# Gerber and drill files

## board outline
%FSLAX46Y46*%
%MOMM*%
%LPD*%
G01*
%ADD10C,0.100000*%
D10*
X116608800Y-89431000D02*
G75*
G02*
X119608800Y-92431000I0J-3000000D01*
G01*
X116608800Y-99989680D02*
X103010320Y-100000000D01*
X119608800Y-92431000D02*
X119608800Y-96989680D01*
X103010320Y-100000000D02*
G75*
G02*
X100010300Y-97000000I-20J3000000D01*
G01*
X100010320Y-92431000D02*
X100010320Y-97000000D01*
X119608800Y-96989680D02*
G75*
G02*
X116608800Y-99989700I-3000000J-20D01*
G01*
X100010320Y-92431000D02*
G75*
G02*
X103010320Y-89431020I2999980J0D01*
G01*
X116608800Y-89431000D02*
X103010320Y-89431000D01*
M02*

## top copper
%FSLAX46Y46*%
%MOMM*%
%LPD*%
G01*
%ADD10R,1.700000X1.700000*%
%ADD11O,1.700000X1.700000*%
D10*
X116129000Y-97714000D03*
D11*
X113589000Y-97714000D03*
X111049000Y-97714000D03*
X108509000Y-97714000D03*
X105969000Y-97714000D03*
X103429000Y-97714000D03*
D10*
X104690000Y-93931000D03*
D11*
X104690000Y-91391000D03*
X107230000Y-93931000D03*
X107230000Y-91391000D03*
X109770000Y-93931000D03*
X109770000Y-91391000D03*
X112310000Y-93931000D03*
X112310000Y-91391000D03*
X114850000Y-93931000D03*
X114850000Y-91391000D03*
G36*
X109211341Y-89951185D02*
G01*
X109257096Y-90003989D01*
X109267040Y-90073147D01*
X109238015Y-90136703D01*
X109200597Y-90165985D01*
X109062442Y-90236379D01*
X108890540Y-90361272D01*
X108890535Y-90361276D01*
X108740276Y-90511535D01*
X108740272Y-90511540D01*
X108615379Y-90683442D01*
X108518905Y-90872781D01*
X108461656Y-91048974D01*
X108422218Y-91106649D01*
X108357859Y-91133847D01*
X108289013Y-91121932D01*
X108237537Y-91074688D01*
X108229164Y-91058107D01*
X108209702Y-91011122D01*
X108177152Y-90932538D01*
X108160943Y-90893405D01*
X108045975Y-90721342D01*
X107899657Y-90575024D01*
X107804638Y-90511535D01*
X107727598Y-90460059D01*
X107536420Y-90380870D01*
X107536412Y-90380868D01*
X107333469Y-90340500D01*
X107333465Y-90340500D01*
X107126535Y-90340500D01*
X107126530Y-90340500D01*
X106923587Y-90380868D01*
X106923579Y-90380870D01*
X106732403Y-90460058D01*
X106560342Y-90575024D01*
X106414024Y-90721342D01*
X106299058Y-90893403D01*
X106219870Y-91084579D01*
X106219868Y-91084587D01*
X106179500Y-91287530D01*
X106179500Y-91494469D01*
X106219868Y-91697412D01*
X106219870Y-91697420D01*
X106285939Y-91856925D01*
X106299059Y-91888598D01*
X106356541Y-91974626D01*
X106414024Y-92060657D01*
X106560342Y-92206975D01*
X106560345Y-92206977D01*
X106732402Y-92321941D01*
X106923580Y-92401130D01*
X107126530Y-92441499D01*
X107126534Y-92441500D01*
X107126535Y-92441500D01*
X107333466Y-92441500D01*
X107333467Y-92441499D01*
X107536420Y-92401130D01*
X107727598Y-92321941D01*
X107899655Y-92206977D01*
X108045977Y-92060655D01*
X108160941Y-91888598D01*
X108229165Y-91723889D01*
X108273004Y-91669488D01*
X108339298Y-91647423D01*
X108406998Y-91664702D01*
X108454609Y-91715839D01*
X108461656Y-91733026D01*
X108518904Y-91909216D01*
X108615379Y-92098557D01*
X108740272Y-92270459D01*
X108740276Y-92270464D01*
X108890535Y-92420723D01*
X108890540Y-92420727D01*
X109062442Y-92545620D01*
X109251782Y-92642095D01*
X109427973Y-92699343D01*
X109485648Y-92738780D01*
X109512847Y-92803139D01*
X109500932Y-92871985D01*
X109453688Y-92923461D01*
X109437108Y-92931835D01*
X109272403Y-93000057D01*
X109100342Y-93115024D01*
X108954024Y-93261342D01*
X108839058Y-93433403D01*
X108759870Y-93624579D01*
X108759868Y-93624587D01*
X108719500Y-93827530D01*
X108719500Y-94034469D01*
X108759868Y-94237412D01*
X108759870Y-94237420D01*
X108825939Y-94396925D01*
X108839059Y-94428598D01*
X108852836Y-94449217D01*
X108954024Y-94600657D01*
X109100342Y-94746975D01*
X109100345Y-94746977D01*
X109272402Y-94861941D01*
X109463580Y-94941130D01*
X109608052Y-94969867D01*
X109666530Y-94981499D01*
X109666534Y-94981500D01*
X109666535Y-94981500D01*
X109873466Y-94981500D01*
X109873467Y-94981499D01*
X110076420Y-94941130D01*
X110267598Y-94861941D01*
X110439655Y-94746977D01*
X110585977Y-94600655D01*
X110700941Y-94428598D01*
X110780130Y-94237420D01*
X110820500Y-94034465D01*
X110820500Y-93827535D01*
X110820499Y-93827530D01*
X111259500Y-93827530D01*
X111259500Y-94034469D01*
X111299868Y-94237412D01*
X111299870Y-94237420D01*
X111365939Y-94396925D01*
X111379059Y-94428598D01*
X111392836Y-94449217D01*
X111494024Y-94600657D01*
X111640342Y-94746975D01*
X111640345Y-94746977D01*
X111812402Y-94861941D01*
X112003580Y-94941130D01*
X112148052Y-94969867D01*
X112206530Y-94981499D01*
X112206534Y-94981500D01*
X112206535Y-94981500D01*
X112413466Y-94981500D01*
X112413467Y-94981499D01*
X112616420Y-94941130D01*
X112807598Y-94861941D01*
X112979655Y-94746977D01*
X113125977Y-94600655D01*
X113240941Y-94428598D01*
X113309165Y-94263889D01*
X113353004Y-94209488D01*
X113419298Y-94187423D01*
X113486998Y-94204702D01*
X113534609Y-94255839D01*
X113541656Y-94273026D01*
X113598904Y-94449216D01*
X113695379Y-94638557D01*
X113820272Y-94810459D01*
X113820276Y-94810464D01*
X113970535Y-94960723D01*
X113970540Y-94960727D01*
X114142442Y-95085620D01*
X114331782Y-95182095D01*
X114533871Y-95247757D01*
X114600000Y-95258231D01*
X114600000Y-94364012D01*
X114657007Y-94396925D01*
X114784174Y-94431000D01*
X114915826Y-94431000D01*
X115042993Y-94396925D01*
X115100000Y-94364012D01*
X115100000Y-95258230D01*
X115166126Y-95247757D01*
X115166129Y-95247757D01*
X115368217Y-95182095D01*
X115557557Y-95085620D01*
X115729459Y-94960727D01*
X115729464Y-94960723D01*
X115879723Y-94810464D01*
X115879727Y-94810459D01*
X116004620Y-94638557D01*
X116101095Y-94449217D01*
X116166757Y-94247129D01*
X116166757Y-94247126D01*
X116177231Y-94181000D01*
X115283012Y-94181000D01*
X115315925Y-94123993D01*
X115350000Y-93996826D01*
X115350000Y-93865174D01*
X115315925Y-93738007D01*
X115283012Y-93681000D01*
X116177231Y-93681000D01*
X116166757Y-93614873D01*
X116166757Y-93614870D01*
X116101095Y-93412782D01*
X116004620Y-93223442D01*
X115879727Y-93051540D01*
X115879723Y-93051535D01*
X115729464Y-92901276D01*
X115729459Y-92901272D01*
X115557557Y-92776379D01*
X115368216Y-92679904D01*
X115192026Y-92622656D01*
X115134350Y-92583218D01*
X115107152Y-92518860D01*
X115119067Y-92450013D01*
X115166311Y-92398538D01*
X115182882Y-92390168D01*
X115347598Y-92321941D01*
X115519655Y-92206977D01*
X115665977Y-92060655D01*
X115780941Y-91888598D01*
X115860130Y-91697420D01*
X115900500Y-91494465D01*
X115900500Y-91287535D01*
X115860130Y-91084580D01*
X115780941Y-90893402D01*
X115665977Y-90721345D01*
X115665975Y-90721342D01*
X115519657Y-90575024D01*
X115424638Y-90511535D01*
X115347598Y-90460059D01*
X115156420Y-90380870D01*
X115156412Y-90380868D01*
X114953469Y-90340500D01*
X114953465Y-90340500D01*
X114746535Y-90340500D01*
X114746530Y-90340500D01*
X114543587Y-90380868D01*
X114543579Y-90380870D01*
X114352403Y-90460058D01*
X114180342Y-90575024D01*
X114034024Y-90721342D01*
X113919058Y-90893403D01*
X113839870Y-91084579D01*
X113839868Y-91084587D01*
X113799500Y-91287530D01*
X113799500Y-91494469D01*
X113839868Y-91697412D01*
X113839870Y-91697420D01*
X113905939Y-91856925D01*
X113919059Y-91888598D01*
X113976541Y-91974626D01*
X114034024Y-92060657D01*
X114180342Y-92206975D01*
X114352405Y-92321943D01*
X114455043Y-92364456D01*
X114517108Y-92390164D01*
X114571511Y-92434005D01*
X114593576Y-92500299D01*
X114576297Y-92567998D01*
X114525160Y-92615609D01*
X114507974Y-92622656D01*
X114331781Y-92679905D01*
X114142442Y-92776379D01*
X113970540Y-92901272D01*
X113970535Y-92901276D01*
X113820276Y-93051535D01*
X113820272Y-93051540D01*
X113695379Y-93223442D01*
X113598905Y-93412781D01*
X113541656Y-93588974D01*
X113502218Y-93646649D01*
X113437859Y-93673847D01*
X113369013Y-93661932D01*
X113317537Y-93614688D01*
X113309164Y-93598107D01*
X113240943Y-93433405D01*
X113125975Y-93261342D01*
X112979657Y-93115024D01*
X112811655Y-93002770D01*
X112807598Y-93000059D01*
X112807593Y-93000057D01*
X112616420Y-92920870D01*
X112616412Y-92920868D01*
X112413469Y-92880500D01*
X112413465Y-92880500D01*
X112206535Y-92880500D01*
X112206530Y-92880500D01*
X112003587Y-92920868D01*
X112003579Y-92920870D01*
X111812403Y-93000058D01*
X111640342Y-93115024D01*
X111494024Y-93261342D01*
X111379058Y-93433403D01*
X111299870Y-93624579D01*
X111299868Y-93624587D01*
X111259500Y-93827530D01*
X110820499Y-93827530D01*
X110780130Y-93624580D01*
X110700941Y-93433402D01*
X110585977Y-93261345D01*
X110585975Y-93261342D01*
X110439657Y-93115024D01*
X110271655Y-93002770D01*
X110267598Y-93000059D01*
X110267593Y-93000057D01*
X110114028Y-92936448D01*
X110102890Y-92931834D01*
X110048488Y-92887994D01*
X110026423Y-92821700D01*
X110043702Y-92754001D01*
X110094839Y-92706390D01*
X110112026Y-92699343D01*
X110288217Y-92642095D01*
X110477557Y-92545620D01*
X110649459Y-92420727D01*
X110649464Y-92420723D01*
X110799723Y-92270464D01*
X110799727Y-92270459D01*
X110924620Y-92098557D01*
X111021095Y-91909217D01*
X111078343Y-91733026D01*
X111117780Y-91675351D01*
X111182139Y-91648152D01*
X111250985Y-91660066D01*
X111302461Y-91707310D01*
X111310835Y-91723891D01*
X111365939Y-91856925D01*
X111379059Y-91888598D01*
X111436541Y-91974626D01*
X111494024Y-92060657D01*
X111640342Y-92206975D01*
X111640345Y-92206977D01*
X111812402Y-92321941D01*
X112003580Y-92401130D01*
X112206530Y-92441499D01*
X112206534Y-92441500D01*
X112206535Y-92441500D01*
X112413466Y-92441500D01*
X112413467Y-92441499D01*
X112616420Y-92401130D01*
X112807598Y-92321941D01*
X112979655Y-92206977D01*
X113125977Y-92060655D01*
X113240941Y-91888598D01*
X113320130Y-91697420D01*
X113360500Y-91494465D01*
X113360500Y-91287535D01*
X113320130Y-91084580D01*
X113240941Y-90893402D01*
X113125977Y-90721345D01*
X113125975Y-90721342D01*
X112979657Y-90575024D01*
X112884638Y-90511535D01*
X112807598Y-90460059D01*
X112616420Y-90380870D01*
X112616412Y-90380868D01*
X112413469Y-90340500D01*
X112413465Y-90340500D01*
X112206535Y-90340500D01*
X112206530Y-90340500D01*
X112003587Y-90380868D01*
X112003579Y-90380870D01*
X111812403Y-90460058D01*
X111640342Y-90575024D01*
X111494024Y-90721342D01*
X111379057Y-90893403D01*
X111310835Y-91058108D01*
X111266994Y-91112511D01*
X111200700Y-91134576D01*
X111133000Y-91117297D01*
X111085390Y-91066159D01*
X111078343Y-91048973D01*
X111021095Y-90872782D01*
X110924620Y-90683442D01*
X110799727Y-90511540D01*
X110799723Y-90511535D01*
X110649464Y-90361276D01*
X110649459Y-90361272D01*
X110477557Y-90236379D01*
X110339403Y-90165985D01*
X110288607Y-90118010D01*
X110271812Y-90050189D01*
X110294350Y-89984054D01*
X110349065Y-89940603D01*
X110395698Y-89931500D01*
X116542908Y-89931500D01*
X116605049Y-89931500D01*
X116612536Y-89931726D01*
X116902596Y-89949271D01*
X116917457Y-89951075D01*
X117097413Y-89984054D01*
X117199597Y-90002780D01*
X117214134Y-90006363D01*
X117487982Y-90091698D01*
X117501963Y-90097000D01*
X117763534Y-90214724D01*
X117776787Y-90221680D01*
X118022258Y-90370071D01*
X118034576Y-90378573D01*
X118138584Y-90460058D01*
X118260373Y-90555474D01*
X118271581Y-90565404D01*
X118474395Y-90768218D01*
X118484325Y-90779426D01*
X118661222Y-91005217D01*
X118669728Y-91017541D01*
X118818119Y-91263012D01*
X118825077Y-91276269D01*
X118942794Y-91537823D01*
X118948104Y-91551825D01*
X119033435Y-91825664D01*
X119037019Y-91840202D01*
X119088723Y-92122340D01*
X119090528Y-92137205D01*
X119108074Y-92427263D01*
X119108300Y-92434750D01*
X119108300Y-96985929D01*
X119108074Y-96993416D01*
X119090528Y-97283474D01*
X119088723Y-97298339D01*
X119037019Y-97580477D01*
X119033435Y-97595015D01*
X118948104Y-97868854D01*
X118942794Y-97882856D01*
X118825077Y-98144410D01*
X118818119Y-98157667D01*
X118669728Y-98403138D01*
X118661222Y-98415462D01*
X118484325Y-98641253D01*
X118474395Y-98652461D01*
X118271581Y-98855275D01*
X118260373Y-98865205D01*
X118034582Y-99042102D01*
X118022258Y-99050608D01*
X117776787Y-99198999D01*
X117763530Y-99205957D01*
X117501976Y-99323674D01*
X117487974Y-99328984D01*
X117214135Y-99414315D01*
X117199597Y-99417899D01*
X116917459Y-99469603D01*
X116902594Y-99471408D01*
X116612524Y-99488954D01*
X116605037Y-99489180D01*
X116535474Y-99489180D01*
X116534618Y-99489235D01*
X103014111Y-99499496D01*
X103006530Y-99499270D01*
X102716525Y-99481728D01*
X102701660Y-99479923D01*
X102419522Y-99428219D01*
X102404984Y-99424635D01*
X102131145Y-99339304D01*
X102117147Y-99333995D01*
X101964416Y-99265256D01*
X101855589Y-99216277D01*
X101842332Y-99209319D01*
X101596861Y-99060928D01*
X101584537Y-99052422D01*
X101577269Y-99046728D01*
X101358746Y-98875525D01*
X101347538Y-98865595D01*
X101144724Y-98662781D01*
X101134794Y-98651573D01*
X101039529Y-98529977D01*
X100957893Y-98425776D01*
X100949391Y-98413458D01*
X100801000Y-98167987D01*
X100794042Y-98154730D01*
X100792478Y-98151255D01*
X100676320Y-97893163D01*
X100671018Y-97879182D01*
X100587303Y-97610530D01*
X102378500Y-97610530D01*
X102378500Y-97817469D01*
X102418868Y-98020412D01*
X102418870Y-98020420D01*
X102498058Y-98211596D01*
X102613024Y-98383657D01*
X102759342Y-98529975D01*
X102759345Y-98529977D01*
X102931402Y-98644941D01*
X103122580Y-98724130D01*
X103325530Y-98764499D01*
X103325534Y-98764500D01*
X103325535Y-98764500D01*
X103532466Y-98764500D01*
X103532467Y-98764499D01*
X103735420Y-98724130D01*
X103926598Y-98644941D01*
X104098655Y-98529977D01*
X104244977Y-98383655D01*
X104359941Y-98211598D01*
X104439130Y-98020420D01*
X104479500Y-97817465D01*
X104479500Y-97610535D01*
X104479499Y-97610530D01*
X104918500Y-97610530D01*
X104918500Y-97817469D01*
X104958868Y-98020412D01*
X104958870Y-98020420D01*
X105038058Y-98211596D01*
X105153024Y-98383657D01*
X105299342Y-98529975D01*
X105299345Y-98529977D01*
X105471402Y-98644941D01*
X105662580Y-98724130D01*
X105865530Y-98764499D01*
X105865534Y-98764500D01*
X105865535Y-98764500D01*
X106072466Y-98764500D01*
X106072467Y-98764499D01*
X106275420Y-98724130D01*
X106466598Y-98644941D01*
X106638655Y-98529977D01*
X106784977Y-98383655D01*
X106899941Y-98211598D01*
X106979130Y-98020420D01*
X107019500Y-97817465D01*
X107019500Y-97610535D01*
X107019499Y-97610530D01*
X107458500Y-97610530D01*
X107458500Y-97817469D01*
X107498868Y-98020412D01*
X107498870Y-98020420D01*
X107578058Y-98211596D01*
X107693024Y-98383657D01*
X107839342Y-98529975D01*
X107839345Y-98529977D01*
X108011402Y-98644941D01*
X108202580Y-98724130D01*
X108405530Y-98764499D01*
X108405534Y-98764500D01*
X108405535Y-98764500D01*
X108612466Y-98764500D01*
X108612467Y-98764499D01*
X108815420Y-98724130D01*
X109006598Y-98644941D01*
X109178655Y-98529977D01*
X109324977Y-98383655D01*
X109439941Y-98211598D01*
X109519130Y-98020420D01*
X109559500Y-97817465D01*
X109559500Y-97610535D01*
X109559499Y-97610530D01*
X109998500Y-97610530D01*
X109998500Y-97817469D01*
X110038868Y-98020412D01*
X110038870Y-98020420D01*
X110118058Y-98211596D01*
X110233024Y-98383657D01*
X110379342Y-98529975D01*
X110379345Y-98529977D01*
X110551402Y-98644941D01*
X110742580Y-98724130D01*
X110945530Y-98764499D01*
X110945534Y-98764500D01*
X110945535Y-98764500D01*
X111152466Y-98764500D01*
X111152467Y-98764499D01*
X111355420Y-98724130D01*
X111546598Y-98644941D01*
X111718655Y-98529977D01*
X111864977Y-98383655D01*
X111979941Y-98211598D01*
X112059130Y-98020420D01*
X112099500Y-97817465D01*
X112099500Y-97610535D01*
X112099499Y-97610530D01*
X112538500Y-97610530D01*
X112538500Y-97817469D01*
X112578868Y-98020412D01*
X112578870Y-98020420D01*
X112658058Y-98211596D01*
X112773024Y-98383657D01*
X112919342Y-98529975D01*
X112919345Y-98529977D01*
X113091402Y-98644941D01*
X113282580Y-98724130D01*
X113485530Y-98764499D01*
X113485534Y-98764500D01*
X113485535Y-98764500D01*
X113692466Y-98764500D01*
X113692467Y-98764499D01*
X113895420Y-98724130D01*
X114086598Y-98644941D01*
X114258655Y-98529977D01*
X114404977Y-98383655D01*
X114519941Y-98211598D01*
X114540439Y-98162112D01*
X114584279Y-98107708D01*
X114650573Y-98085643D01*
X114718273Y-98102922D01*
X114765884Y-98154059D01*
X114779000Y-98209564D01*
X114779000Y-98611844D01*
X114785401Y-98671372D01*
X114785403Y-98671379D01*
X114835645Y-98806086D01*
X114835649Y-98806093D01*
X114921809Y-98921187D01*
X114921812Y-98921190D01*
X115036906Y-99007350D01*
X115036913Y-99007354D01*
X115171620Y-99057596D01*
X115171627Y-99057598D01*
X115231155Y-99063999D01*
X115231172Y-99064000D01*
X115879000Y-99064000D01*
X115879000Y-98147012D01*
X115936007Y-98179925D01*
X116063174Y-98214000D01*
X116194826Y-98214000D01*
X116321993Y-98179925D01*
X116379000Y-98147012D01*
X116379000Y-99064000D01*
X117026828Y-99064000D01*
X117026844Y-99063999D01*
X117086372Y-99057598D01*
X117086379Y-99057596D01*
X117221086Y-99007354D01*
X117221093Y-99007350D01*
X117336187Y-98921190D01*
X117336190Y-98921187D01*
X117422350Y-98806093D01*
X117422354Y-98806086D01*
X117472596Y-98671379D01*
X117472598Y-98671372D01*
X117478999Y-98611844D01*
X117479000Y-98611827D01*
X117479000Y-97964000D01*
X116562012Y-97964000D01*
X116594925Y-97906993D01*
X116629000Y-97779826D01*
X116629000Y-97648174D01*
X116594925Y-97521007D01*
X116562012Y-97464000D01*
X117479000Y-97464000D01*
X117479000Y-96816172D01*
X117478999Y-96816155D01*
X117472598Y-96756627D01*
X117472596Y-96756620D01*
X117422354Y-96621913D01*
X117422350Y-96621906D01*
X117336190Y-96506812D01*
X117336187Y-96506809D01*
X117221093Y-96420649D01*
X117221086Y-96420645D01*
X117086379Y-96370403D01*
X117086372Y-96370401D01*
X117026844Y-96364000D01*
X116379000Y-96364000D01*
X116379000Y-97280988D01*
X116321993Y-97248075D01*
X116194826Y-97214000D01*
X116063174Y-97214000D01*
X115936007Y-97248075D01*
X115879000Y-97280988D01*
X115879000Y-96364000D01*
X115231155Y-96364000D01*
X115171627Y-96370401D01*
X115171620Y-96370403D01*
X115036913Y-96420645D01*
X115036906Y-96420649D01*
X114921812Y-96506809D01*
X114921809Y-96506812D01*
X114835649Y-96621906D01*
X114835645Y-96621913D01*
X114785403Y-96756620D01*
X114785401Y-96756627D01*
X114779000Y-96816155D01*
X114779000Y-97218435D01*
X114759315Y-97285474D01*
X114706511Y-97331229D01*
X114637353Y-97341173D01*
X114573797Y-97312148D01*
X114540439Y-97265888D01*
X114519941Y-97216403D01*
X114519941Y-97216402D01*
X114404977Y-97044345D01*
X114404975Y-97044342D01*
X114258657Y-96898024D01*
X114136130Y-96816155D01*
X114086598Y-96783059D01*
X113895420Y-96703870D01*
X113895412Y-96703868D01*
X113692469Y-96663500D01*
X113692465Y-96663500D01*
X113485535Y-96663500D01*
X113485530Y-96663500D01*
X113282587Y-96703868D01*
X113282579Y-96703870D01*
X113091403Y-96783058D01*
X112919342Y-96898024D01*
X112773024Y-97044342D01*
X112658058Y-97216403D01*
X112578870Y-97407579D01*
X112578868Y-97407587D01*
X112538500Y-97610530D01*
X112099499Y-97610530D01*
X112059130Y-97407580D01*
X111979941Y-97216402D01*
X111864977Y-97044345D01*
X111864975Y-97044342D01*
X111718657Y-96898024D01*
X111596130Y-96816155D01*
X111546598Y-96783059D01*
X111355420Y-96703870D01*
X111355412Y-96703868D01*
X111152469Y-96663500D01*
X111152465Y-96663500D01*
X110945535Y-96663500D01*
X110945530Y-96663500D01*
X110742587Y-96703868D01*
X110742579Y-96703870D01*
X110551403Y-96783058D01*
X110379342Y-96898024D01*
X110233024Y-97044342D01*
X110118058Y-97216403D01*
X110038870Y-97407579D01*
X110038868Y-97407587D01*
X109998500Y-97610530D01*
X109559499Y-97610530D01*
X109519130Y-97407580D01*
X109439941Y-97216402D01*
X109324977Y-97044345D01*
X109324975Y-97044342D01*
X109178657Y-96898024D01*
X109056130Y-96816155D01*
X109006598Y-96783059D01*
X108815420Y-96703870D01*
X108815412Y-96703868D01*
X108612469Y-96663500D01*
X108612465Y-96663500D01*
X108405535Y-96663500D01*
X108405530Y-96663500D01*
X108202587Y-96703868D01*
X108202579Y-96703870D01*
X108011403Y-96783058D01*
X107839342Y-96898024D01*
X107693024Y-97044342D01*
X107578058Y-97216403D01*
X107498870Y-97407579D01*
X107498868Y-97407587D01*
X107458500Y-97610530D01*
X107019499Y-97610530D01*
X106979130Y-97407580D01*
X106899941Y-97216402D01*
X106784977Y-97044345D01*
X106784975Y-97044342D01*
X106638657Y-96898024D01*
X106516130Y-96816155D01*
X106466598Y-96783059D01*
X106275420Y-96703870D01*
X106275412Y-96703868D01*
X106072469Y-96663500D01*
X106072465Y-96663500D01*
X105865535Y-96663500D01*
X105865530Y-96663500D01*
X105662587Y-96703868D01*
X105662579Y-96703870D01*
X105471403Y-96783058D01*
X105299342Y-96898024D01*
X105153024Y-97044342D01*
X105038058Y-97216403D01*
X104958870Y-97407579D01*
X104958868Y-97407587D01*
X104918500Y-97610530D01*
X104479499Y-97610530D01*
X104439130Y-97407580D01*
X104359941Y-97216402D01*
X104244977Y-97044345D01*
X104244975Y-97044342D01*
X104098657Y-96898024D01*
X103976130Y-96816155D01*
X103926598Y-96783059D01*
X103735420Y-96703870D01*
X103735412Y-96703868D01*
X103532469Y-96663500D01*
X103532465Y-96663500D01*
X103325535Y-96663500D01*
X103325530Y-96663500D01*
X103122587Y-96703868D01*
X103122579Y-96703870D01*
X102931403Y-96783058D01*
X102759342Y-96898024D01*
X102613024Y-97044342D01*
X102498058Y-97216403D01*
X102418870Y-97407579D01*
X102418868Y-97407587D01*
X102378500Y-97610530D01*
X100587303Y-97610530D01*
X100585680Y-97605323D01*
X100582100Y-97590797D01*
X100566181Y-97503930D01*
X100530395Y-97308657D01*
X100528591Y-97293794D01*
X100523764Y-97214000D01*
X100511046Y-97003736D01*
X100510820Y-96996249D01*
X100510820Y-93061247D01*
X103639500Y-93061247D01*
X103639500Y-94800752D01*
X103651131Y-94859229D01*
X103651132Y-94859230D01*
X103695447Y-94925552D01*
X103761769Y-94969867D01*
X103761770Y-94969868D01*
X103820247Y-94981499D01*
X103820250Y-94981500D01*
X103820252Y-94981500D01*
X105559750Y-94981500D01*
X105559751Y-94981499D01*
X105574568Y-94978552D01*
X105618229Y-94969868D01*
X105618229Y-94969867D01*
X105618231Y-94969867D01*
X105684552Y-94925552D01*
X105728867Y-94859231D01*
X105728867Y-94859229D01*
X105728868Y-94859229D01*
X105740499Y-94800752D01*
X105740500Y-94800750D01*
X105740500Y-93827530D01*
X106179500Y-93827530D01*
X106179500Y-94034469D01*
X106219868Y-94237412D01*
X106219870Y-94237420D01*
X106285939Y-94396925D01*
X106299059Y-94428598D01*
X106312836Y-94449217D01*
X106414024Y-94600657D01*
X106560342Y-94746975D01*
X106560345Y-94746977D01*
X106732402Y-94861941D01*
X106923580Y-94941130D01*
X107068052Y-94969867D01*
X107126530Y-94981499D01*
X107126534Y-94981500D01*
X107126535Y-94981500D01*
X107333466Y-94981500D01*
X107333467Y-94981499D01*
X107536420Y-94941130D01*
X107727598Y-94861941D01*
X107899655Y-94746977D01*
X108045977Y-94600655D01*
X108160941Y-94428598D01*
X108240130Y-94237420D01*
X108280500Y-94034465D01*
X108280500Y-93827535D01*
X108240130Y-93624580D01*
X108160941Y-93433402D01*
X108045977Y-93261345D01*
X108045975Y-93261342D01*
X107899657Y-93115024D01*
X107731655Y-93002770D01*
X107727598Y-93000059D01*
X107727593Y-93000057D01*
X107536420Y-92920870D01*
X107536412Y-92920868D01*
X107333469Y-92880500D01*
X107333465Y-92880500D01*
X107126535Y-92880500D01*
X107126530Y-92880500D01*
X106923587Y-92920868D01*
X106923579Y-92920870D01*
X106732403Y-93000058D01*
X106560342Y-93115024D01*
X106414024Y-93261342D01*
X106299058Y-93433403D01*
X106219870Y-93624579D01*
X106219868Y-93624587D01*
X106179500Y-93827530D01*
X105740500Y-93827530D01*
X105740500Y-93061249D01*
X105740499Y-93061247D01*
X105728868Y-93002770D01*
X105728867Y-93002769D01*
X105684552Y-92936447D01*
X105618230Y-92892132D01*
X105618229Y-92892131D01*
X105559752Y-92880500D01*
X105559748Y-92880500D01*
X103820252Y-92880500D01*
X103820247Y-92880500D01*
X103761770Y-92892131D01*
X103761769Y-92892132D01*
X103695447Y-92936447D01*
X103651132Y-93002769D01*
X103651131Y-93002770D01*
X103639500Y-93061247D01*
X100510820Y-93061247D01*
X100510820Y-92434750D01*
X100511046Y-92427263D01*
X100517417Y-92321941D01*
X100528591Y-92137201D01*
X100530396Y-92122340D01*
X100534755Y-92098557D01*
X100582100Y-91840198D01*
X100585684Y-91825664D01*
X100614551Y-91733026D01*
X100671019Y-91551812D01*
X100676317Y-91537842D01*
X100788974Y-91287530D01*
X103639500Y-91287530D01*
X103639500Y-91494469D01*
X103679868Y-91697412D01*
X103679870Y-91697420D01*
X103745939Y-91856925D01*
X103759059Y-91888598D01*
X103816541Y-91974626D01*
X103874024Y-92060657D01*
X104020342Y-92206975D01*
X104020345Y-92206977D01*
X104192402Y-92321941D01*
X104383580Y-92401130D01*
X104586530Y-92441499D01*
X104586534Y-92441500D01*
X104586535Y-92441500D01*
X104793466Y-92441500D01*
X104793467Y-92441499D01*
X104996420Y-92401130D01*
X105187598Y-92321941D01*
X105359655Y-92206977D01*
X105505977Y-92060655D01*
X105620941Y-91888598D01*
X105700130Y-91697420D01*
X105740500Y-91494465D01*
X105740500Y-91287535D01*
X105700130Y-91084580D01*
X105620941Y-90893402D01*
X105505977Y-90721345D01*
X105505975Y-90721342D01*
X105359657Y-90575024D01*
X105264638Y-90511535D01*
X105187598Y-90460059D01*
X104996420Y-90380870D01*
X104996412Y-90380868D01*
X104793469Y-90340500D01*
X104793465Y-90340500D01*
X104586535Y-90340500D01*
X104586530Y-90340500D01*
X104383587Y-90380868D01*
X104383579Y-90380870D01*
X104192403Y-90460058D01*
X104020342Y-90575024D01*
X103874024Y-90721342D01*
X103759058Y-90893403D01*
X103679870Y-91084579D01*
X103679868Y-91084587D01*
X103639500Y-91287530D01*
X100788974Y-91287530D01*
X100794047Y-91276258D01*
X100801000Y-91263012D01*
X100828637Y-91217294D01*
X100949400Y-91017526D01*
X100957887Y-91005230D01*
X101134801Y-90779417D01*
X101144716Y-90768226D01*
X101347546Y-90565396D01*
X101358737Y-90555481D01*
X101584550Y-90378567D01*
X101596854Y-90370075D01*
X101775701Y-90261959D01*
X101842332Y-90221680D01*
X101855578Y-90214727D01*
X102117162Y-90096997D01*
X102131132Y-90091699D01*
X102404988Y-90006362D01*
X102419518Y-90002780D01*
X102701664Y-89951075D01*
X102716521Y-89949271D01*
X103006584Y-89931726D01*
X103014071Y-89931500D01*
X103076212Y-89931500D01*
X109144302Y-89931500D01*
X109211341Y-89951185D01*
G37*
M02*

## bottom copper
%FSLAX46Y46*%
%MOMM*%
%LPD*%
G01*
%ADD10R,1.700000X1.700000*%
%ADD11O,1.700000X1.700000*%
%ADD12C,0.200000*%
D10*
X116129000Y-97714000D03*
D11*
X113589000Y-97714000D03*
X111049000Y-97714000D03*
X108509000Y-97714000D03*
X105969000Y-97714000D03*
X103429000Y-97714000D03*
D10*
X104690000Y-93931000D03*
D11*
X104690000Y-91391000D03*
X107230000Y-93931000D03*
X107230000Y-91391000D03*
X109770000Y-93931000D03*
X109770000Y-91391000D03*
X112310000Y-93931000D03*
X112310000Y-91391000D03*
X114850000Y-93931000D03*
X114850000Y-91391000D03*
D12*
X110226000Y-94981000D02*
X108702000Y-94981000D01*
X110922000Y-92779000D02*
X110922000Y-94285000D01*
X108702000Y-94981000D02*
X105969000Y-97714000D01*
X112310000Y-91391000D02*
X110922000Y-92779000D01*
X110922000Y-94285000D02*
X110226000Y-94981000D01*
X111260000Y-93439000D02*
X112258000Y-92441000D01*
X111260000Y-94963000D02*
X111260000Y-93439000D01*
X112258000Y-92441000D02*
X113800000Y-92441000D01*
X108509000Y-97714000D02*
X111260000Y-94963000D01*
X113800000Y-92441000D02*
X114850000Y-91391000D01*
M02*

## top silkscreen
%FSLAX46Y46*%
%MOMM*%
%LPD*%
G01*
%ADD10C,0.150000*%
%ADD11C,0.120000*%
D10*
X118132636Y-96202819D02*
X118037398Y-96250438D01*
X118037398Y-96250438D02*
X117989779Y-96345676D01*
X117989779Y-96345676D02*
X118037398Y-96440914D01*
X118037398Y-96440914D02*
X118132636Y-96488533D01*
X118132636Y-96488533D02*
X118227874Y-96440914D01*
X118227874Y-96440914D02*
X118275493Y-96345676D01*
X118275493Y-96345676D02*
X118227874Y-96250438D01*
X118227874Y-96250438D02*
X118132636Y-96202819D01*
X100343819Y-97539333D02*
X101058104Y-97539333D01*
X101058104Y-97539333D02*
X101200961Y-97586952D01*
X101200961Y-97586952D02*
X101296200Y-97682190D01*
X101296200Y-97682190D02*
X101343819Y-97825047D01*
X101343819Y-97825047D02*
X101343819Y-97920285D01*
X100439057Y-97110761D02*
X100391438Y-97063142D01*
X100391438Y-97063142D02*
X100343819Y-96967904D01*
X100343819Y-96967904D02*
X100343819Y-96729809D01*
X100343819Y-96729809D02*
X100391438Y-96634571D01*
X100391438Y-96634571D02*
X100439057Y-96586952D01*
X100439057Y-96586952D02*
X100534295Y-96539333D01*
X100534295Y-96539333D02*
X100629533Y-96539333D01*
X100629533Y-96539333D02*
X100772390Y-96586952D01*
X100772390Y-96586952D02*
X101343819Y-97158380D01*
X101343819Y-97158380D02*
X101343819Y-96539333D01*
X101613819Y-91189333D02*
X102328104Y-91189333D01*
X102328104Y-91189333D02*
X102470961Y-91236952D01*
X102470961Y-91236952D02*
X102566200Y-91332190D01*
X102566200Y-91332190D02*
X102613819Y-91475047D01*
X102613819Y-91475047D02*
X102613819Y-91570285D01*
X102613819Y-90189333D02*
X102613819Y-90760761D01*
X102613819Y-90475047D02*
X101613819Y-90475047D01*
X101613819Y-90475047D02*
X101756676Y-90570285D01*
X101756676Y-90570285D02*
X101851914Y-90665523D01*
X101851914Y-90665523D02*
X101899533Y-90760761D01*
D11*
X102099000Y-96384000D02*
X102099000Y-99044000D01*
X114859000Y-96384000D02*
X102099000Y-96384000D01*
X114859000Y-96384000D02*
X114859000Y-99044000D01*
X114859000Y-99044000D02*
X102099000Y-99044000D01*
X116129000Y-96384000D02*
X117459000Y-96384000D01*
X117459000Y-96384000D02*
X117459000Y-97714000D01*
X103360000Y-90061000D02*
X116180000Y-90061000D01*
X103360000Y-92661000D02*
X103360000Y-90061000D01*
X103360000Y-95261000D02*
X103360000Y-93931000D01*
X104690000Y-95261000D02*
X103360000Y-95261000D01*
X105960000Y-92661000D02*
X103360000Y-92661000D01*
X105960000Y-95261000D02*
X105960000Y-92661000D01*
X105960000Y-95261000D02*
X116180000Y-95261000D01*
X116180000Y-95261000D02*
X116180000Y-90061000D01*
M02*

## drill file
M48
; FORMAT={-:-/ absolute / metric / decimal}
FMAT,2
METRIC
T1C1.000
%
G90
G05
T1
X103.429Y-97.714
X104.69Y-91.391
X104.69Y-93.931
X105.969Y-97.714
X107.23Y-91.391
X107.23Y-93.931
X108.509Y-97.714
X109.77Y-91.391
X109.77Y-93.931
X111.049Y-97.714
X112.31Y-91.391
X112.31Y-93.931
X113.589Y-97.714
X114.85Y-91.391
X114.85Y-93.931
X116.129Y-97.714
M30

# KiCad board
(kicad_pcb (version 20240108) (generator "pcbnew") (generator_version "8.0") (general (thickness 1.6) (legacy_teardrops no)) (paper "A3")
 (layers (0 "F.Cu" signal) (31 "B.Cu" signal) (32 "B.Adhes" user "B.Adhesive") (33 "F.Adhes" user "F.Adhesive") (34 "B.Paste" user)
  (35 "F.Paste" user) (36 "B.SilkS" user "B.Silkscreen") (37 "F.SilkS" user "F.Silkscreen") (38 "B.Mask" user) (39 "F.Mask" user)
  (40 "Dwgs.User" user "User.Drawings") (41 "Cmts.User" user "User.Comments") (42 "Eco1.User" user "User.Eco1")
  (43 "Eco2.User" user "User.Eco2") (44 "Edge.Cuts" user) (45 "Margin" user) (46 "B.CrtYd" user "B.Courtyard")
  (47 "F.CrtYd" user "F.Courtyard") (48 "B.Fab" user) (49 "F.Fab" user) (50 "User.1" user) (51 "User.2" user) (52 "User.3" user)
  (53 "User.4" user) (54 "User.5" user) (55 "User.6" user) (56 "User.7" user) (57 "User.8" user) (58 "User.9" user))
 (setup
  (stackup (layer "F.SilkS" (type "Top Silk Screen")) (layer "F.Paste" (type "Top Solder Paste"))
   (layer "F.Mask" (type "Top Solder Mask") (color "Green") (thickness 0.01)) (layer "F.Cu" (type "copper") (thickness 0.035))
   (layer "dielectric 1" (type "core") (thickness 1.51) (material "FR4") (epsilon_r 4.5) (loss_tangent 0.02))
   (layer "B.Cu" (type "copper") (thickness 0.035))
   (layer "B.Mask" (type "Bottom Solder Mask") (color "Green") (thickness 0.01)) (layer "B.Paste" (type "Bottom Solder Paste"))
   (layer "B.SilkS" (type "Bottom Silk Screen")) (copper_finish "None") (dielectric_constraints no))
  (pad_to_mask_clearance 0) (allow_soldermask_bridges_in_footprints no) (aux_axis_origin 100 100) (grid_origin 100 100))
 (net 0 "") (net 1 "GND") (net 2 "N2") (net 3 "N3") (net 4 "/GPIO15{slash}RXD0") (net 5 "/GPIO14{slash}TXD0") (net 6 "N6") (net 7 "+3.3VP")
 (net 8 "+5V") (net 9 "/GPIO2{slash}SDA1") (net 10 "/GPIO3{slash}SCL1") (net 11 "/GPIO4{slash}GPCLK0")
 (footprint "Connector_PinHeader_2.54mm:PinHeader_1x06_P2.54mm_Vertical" (layer "F.Cu") (at 116.129 97.714 -90)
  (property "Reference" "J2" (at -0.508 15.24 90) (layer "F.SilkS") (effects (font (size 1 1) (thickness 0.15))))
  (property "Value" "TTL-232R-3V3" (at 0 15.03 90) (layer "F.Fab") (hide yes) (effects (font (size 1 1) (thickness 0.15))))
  (fp_line (start -1.33 14.03) (end 1.33 14.03) (stroke (width 0.12) (type solid)) (layer "F.SilkS"))
  (fp_line (start -1.33 1.27) (end -1.33 14.03) (stroke (width 0.12) (type solid)) (layer "F.SilkS"))
  (fp_line (start -1.33 1.27) (end 1.33 1.27) (stroke (width 0.12) (type solid)) (layer "F.SilkS"))
  (fp_line (start 1.33 1.27) (end 1.33 14.03) (stroke (width 0.12) (type solid)) (layer "F.SilkS"))
  (fp_line (start -1.33 0) (end -1.33 -1.33) (stroke (width 0.12) (type solid)) (layer "F.SilkS"))
  (fp_line (start -1.33 -1.33) (end 0 -1.33) (stroke (width 0.12) (type solid)) (layer "F.SilkS"))
  (pad "1" thru_hole rect (at 0 0 270) (size 1.7 1.7) (drill 1) (layers "*.Cu" "*.Mask") (remove_unused_layers no) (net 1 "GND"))
  (pad "2" thru_hole oval (at 0 2.54 270) (size 1.7 1.7) (drill 1) (layers "*.Cu" "*.Mask") (remove_unused_layers no) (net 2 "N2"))
  (pad "3" thru_hole oval (at 0 5.08 270) (size 1.7 1.7) (drill 1) (layers "*.Cu" "*.Mask") (remove_unused_layers no) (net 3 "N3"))
  (pad "4" thru_hole oval (at 0 7.62 270) (size 1.7 1.7) (drill 1) (layers "*.Cu" "*.Mask") (remove_unused_layers no)
   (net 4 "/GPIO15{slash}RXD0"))
  (pad "5" thru_hole oval (at 0 10.16 270) (size 1.7 1.7) (drill 1) (layers "*.Cu" "*.Mask") (remove_unused_layers no)
   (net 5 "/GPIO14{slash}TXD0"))
  (pad "6" thru_hole oval (at 0 12.7 270) (size 1.7 1.7) (drill 1) (layers "*.Cu" "*.Mask") (remove_unused_layers no) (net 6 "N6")))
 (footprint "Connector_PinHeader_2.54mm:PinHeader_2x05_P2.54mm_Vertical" (layer "F.Cu") (at 104.69 93.931 90)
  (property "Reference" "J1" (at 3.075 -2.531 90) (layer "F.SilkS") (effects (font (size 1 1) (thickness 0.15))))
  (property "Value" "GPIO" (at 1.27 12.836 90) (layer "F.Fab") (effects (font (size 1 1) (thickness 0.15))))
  (fp_line (start 3.87 -1.33) (end 3.87 11.49) (stroke (width 0.12) (type solid)) (layer "F.SilkS"))
  (fp_line (start 1.27 -1.33) (end 3.87 -1.33) (stroke (width 0.12) (type solid)) (layer "F.SilkS"))
  (fp_line (start -1.33 -1.33) (end 0 -1.33) (stroke (width 0.12) (type solid)) (layer "F.SilkS"))
  (fp_line (start -1.33 0) (end -1.33 -1.33) (stroke (width 0.12) (type solid)) (layer "F.SilkS"))
  (fp_line (start 1.27 1.27) (end 1.27 -1.33) (stroke (width 0.12) (type solid)) (layer "F.SilkS"))
  (fp_line (start -1.33 1.27) (end 1.27 1.27) (stroke (width 0.12) (type solid)) (layer "F.SilkS"))
  (fp_line (start -1.33 1.27) (end -1.33 11.49) (stroke (width 0.12) (type solid)) (layer "F.SilkS"))
  (fp_line (start -1.33 11.49) (end 3.87 11.49) (stroke (width 0.12) (type solid)) (layer "F.SilkS"))
  (pad "1" thru_hole rect (at 0 0 90) (size 1.7 1.7) (drill 1) (layers "*.Cu" "*.Mask") (remove_unused_layers no) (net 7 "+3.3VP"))
  (pad "2" thru_hole oval (at 2.54 0 90) (size 1.7 1.7) (drill 1) (layers "*.Cu" "*.Mask") (remove_unused_layers no) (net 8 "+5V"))
  (pad "3" thru_hole oval (at 0 2.54 90) (size 1.7 1.7) (drill 1) (layers "*.Cu" "*.Mask") (remove_unused_layers no)
   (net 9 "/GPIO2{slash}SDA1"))
  (pad "4" thru_hole oval (at 2.54 2.54 90) (size 1.7 1.7) (drill 1) (layers "*.Cu" "*.Mask") (remove_unused_layers no) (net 8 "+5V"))
  (pad "5" thru_hole oval (at 0 5.08 90) (size 1.7 1.7) (drill 1) (layers "*.Cu" "*.Mask") (remove_unused_layers no)
   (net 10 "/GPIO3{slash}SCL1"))
  (pad "6" thru_hole oval (at 2.54 5.08 90) (size 1.7 1.7) (drill 1) (layers "*.Cu" "*.Mask") (remove_unused_layers no) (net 1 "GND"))
  (pad "7" thru_hole oval (at 0 7.62 90) (size 1.7 1.7) (drill 1) (layers "*.Cu" "*.Mask") (remove_unused_layers no)
   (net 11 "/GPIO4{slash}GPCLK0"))
  (pad "8" thru_hole oval (at 2.54 7.62 90) (size 1.7 1.7) (drill 1) (layers "*.Cu" "*.Mask") (remove_unused_layers no)
   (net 5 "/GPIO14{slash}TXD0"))
  (pad "9" thru_hole oval (at 0 10.16 90) (size 1.7 1.7) (drill 1) (layers "*.Cu" "*.Mask") (remove_unused_layers no) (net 1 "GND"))
  (pad "10" thru_hole oval (at 2.54 10.16 90) (size 1.7 1.7) (drill 1) (layers "*.Cu" "*.Mask") (remove_unused_layers no)
   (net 4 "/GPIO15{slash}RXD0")))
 (gr_arc (start 116.6088 89.431) (mid 118.73012 90.30968) (end 119.6088 92.431) (stroke (width 0.1) (type solid)) (layer "Edge.Cuts"))
 (gr_line (start 116.6088 99.98968) (end 103.01032 100) (stroke (width 0.1) (type solid)) (layer "Edge.Cuts"))
 (gr_line (start 119.6088 92.431) (end 119.6088 96.98968) (stroke (width 0.1) (type solid)) (layer "Edge.Cuts"))
 (gr_arc (start 103.01032 100) (mid 100.889 99.12132) (end 100.01032 97) (stroke (width 0.1) (type solid)) (layer "Edge.Cuts"))
 (gr_line (start 100.01032 92.431) (end 100.01032 97) (stroke (width 0.1) (type solid)) (layer "Edge.Cuts"))
 (gr_arc (start 119.6088 96.98968) (mid 118.73012 99.111) (end 116.6088 99.98968) (stroke (width 0.1) (type solid)) (layer "Edge.Cuts"))
 (gr_arc (start 100.01032 92.431) (mid 100.889 90.30968) (end 103.01032 89.431) (stroke (width 0.1) (type solid)) (layer "Edge.Cuts"))
 (gr_line (start 116.6088 89.431) (end 103.01032 89.431) (stroke (width 0.1) (type solid)) (layer "Edge.Cuts"))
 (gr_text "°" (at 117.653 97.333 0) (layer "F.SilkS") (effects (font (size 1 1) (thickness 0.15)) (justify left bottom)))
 (segment (start 110.226 94.981) (end 108.702 94.981) (width 0.2) (layer "B.Cu") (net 5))
 (segment (start 110.922 92.779) (end 110.922 94.285) (width 0.2) (layer "B.Cu") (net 5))
 (segment (start 108.702 94.981) (end 105.969 97.714) (width 0.2) (layer "B.Cu") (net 5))
 (segment (start 112.31 91.391) (end 110.922 92.779) (width 0.2) (layer "B.Cu") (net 5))
 (segment (start 110.922 94.285) (end 110.226 94.981) (width 0.2) (layer "B.Cu") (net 5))
 (segment (start 111.26 93.439) (end 112.258 92.441) (width 0.2) (layer "B.Cu") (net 4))
 (segment (start 111.26 94.963) (end 111.26 93.439) (width 0.2) (layer "B.Cu") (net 4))
 (segment (start 112.258 92.441) (end 113.8 92.441) (width 0.2) (layer "B.Cu") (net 4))
 (segment (start 108.509 97.714) (end 111.26 94.963) (width 0.2) (layer "B.Cu") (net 4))
 (segment (start 113.8 92.441) (end 114.85 91.391) (width 0.2) (layer "B.Cu") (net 4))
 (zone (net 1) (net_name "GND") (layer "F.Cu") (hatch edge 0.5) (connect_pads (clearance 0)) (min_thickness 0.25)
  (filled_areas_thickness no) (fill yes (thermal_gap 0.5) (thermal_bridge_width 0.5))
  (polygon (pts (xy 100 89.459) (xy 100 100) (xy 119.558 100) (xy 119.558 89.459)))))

